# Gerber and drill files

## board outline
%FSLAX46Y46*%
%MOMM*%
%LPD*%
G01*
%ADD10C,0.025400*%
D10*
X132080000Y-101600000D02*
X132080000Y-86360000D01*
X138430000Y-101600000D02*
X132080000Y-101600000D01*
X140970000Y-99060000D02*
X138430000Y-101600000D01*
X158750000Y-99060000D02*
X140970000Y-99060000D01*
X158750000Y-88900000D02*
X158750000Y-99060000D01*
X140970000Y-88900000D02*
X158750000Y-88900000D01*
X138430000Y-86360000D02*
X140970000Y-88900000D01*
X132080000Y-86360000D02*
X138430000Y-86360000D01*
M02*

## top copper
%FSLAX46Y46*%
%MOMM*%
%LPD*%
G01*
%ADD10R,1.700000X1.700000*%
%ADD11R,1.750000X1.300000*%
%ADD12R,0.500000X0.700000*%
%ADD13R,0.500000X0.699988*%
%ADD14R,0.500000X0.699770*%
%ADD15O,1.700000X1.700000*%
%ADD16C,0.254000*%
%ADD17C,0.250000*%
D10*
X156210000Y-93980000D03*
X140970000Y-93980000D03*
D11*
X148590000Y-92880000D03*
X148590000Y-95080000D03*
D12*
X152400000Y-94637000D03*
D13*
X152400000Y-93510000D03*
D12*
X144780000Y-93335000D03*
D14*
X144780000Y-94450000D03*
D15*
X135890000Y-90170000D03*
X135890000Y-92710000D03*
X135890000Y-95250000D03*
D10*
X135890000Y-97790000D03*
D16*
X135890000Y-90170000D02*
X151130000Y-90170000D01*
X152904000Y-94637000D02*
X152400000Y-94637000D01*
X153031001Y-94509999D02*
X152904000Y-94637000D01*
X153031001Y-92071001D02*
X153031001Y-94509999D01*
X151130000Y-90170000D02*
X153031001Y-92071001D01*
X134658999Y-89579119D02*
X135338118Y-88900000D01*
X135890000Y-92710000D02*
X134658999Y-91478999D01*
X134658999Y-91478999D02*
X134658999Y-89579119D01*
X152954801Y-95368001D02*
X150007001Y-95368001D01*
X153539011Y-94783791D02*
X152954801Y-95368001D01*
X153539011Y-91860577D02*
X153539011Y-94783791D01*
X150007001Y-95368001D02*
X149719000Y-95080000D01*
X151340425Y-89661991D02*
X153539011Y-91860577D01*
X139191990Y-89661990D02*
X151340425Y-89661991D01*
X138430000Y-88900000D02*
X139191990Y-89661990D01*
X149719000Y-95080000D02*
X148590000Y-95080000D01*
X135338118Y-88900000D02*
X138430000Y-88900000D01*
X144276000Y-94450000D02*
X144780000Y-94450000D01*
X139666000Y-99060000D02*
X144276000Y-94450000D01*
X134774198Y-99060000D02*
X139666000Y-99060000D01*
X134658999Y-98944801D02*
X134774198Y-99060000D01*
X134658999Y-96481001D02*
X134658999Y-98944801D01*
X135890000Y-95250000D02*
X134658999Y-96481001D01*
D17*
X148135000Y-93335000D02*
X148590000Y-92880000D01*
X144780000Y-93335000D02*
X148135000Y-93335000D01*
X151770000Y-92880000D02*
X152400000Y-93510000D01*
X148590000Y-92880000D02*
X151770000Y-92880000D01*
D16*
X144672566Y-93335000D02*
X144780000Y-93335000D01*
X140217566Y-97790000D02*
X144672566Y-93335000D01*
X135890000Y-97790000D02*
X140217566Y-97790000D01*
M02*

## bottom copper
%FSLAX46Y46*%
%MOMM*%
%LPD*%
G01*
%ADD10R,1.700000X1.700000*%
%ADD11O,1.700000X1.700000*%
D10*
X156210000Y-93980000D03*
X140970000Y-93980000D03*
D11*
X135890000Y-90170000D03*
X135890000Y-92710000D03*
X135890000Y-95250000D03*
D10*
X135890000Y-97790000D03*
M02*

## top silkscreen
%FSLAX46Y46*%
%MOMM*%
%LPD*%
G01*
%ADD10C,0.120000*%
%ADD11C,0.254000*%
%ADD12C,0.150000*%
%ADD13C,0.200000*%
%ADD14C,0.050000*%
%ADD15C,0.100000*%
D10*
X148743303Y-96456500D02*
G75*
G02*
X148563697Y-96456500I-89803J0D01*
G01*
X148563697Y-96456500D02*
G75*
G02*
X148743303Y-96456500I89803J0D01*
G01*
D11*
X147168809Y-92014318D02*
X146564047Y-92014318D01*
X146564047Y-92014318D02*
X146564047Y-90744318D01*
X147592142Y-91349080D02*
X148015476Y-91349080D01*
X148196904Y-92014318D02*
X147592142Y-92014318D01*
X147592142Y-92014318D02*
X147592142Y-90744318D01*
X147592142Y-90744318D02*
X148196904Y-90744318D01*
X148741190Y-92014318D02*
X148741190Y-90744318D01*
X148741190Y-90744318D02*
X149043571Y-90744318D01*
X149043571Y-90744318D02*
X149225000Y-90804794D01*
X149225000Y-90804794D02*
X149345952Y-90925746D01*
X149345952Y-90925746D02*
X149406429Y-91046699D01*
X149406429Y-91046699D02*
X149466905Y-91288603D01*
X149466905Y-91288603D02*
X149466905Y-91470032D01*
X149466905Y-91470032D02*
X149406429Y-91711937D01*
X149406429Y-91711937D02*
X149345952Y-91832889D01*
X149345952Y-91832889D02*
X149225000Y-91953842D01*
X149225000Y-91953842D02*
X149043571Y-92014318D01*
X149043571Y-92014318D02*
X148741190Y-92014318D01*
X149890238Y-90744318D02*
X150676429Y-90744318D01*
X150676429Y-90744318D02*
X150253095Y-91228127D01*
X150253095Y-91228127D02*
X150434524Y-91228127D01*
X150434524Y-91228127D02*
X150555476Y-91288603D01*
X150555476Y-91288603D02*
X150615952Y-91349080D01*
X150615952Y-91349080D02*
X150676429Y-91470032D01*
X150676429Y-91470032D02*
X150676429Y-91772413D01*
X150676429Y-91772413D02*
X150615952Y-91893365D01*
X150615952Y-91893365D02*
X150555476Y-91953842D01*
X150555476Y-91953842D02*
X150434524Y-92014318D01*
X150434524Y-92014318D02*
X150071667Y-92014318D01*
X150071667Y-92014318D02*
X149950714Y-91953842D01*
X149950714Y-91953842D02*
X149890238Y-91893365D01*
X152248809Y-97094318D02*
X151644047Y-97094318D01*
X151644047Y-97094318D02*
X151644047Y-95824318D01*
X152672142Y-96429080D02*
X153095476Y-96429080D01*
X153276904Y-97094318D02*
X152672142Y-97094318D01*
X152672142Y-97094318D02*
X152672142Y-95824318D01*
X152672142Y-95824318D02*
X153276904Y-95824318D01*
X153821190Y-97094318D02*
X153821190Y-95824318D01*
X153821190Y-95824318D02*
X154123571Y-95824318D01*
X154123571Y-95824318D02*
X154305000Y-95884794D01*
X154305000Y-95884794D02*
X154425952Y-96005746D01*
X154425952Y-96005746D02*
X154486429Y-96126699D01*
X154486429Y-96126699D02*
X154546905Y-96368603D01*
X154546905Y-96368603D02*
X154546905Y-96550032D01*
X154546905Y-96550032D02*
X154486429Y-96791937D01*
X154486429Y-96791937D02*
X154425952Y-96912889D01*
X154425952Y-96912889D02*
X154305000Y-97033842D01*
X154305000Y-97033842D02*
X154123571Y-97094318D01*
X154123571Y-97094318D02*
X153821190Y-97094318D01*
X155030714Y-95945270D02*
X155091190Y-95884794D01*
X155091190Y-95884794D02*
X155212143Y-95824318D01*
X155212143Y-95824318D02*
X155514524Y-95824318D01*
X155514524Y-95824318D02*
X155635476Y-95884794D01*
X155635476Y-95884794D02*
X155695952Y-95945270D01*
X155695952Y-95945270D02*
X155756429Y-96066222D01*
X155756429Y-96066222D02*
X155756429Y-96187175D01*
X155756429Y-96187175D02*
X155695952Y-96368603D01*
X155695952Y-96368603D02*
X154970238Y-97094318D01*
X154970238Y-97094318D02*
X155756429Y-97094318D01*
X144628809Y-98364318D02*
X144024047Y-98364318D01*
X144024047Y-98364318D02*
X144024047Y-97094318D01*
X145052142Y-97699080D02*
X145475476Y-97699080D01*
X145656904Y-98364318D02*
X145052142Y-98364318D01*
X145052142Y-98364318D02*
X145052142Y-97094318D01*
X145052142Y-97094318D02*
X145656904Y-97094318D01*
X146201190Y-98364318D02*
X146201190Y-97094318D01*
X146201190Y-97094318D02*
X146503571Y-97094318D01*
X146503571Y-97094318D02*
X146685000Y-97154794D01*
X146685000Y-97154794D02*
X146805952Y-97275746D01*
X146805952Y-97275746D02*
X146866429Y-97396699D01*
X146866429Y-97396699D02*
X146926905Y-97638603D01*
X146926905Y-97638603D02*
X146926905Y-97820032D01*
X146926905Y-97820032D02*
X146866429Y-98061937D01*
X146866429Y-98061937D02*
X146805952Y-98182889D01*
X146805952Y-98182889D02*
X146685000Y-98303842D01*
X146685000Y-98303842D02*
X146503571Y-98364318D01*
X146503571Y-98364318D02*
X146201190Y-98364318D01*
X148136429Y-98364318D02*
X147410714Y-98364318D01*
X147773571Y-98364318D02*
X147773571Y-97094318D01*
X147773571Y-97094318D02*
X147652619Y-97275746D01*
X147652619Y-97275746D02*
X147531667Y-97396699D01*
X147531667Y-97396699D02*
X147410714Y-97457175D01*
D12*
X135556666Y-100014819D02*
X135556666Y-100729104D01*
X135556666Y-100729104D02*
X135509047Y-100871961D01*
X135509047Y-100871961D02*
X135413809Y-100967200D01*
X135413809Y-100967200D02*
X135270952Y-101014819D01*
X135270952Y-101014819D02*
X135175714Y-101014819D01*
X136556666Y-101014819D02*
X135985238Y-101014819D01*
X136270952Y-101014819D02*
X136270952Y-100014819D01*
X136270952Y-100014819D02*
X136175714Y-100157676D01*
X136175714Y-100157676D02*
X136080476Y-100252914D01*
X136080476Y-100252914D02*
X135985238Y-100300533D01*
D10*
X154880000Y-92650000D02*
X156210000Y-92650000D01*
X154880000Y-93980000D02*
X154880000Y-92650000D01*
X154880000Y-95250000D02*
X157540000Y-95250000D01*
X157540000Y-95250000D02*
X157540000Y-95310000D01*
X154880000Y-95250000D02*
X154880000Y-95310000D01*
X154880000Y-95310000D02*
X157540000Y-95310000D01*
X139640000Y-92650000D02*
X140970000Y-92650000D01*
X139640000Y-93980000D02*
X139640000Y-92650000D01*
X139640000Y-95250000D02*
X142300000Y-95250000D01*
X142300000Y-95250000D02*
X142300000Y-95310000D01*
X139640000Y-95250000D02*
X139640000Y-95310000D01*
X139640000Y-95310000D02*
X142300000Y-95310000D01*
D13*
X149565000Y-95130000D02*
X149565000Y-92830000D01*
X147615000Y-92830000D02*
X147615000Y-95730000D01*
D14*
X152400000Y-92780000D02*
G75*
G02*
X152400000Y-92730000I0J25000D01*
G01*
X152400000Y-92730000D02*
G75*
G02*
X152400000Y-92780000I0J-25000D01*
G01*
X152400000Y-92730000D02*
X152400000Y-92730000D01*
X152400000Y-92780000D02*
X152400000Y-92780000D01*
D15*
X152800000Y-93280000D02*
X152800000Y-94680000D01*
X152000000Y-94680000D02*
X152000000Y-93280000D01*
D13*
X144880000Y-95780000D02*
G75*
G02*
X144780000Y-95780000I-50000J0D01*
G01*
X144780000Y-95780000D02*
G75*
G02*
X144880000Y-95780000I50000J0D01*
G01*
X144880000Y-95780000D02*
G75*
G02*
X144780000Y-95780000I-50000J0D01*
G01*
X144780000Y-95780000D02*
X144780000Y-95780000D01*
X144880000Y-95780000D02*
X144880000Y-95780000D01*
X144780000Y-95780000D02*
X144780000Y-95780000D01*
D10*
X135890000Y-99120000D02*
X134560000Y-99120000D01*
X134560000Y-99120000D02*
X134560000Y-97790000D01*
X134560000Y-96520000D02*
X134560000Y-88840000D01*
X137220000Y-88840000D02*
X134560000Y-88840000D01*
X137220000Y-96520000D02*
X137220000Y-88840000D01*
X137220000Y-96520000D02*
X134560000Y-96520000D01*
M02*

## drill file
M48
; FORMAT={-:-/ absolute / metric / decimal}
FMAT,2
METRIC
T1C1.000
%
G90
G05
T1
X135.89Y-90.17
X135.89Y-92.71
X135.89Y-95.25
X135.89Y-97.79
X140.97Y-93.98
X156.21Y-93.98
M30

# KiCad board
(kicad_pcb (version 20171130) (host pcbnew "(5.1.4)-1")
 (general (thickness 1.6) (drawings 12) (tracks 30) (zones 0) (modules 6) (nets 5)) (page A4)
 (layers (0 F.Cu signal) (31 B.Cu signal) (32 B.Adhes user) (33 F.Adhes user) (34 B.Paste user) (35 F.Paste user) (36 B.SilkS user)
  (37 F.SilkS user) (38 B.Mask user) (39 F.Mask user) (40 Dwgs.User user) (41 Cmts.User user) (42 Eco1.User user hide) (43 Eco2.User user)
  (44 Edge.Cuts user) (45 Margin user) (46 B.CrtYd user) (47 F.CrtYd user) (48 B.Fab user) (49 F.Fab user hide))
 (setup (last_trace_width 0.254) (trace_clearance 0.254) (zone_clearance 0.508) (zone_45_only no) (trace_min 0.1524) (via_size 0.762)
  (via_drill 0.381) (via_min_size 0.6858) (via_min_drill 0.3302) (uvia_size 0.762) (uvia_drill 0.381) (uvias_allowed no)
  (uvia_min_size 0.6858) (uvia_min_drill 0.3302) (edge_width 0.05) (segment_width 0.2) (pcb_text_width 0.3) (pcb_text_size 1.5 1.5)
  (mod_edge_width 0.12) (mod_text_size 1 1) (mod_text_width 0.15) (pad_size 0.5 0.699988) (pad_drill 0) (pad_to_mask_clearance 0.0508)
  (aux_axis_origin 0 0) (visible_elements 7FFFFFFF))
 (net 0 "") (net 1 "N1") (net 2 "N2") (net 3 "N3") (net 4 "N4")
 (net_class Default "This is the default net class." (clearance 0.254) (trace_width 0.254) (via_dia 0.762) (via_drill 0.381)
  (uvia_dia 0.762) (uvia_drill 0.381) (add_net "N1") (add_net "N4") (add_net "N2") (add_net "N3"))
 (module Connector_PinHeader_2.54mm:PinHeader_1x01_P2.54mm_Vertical (layer F.Cu) (at 156.21 93.98)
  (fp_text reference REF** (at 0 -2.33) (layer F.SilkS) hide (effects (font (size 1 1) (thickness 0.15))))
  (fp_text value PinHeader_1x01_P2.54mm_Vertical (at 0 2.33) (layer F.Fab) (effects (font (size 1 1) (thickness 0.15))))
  (fp_line (start -1.33 -1.33) (end 0 -1.33) (layer F.SilkS) (width 0.12))
  (fp_line (start -1.33 0) (end -1.33 -1.33) (layer F.SilkS) (width 0.12))
  (fp_line (start -1.33 1.27) (end 1.33 1.27) (layer F.SilkS) (width 0.12))
  (fp_line (start 1.33 1.27) (end 1.33 1.33) (layer F.SilkS) (width 0.12))
  (fp_line (start -1.33 1.27) (end -1.33 1.33) (layer F.SilkS) (width 0.12))
  (fp_line (start -1.33 1.33) (end 1.33 1.33) (layer F.SilkS) (width 0.12))
  (pad 1 thru_hole rect (at 0 0) (size 1.7 1.7) (drill 1) (layers *.Cu *.Mask)))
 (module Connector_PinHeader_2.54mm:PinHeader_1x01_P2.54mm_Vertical (layer F.Cu) (at 140.97 93.98)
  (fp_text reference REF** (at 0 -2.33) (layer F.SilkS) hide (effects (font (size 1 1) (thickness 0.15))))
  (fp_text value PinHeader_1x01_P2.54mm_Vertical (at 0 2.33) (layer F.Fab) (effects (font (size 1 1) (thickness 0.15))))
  (fp_line (start -1.33 -1.33) (end 0 -1.33) (layer F.SilkS) (width 0.12))
  (fp_line (start -1.33 0) (end -1.33 -1.33) (layer F.SilkS) (width 0.12))
  (fp_line (start -1.33 1.27) (end 1.33 1.27) (layer F.SilkS) (width 0.12))
  (fp_line (start 1.33 1.27) (end 1.33 1.33) (layer F.SilkS) (width 0.12))
  (fp_line (start -1.33 1.27) (end -1.33 1.33) (layer F.SilkS) (width 0.12))
  (fp_line (start -1.33 1.33) (end 1.33 1.33) (layer F.SilkS) (width 0.12))
  (pad 1 thru_hole rect (at 0 0) (size 1.7 1.7) (drill 1) (layers *.Cu *.Mask)))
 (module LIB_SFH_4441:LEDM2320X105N (layer F.Cu) (at 148.59 93.98 90)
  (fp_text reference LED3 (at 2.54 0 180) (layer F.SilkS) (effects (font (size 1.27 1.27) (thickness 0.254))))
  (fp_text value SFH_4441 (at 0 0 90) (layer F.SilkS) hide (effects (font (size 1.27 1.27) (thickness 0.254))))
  (fp_line (start -1.15 0.975) (end 1.15 0.975) (layer F.SilkS) (width 0.2))
  (fp_line (start 1.15 -0.975) (end -1.75 -0.975) (layer F.SilkS) (width 0.2))
  (pad 2 smd rect (at 1.1 0 90) (size 1.3 1.75) (layers F.Cu F.Paste F.Mask) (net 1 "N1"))
  (pad 1 smd rect (at -1.1 0 90) (size 1.3 1.75) (layers F.Cu F.Paste F.Mask) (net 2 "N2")))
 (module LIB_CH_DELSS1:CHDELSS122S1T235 (layer F.Cu) (at 152.4 93.98 90)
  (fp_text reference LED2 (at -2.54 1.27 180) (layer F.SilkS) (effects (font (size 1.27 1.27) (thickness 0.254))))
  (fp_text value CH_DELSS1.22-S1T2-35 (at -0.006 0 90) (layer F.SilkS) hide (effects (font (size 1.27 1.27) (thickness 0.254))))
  (fp_arc (start 1.225 0) (end 1.25 0) (angle -180) (layer F.SilkS) (width 0.05))
  (fp_arc (start 1.225 0) (end 1.2 0) (angle -180) (layer F.SilkS) (width 0.05))
  (fp_line (start 1.25 0) (end 1.25 0) (layer F.SilkS) (width 0.05))
  (fp_line (start 1.2 0) (end 1.2 0) (layer F.SilkS) (width 0.05))
  (fp_line (start 0.7 0.4) (end -0.7 0.4) (layer F.SilkS) (width 0.1))
  (fp_line (start -0.7 -0.4) (end 0.7 -0.4) (layer F.SilkS) (width 0.1))
  (pad 2 smd rect (at -0.657 0 180) (size 0.5 0.7) (layers F.Cu F.Paste F.Mask) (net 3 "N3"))
  (pad 1 smd rect (at 0.47 0 180) (size 0.5 0.699988) (layers F.Cu F.Paste F.Mask) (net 1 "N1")))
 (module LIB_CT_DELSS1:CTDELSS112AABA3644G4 (layer F.Cu) (at 144.78 93.98)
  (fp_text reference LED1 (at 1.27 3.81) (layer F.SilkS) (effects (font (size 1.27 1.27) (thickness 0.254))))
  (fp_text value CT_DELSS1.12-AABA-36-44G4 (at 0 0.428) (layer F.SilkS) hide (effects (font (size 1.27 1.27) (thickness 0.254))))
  (fp_arc (start 0.05 1.8) (end 0 1.8) (angle -180) (layer F.SilkS) (width 0.2))
  (fp_arc (start 0.05 1.8) (end 0.1 1.8) (angle -180) (layer F.SilkS) (width 0.2))
  (fp_arc (start 0.05 1.8) (end 0 1.8) (angle -180) (layer F.SilkS) (width 0.2))
  (fp_line (start 0 1.8) (end 0 1.8) (layer F.SilkS) (width 0.2))
  (fp_line (start 0.1 1.8) (end 0.1 1.8) (layer F.SilkS) (width 0.2))
  (fp_line (start 0 1.8) (end 0 1.8) (layer F.SilkS) (width 0.2))
  (pad 2 smd rect (at 0 -0.645) (size 0.5 0.7) (layers F.Cu F.Paste F.Mask) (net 1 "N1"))
  (pad 1 smd rect (at 0 0.47) (size 0.5 0.69977) (layers F.Cu F.Paste F.Mask) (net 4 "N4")))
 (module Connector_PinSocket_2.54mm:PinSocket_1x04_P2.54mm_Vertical (layer F.Cu) (at 135.89 97.79 180)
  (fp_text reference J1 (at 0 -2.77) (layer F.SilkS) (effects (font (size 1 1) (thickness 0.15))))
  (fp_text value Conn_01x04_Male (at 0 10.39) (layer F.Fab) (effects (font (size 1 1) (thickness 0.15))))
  (fp_line (start 0 -1.33) (end 1.33 -1.33) (layer F.SilkS) (width 0.12))
  (fp_line (start 1.33 -1.33) (end 1.33 0) (layer F.SilkS) (width 0.12))
  (fp_line (start 1.33 1.27) (end 1.33 8.95) (layer F.SilkS) (width 0.12))
  (fp_line (start -1.33 8.95) (end 1.33 8.95) (layer F.SilkS) (width 0.12))
  (fp_line (start -1.33 1.27) (end -1.33 8.95) (layer F.SilkS) (width 0.12))
  (fp_line (start -1.33 1.27) (end 1.33 1.27) (layer F.SilkS) (width 0.12))
  (pad 4 thru_hole oval (at 0 7.62 180) (size 1.7 1.7) (drill 1) (layers *.Cu *.Mask) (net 3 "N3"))
  (pad 3 thru_hole oval (at 0 5.08 180) (size 1.7 1.7) (drill 1) (layers *.Cu *.Mask) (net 2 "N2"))
  (pad 2 thru_hole oval (at 0 2.54 180) (size 1.7 1.7) (drill 1) (layers *.Cu *.Mask) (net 4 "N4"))
  (pad 1 thru_hole rect (at 0 0 180) (size 1.7 1.7) (drill 1) (layers *.Cu *.Mask) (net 1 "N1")))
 (gr_circle (center 148.6535 96.4565) (end 148.717 96.52) (layer F.SilkS) (width 0.12))
 (gr_line (start 132.08 101.6) (end 132.08 86.36) (layer Edge.Cuts) (width 0.0254))
 (gr_line (start 138.43 101.6) (end 132.08 101.6) (layer Edge.Cuts) (width 0.0254))
 (gr_line (start 140.97 99.06) (end 138.43 101.6) (layer Edge.Cuts) (width 0.0254))
 (gr_line (start 158.75 99.06) (end 140.97 99.06) (layer Edge.Cuts) (width 0.0254))
 (gr_line (start 158.75 88.9) (end 158.75 99.06) (layer Edge.Cuts) (width 0.0254))
 (gr_line (start 140.97 88.9) (end 158.75 88.9) (layer Edge.Cuts) (width 0.0254))
 (gr_line (start 138.43 86.36) (end 140.97 88.9) (layer Edge.Cuts) (width 0.0254))
 (gr_line (start 132.08 86.36) (end 138.43 86.36) (layer Edge.Cuts) (width 0.0254))
 (segment (start 135.89 90.17) (end 151.13 90.17) (width 0.254) (layer F.Cu) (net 3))
 (segment (start 152.904 94.637) (end 152.4 94.637) (width 0.254) (layer F.Cu) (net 3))
 (segment (start 153.031001 94.509999) (end 152.904 94.637) (width 0.254) (layer F.Cu) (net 3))
 (segment (start 153.031001 92.071001) (end 153.031001 94.509999) (width 0.254) (layer F.Cu) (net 3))
 (segment (start 151.13 90.17) (end 153.031001 92.071001) (width 0.254) (layer F.Cu) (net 3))
 (segment (start 134.658999 89.579119) (end 135.338118 88.9) (width 0.254) (layer F.Cu) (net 2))
 (segment (start 135.89 92.71) (end 134.658999 91.478999) (width 0.254) (layer F.Cu) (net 2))
 (segment (start 134.658999 91.478999) (end 134.658999 89.579119) (width 0.254) (layer F.Cu) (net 2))
 (segment (start 152.954801 95.368001) (end 150.007001 95.368001) (width 0.254) (layer F.Cu) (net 2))
 (segment (start 153.539011 94.783791) (end 152.954801 95.368001) (width 0.254) (layer F.Cu) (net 2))
 (segment (start 153.539011 91.860577) (end 153.539011 94.783791) (width 0.254) (layer F.Cu) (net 2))
 (segment (start 150.007001 95.368001) (end 149.719 95.08) (width 0.254) (layer F.Cu) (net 2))
 (segment (start 151.340425 89.661991) (end 153.539011 91.860577) (width 0.254) (layer F.Cu) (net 2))
 (segment (start 139.19199 89.66199) (end 151.340425 89.661991) (width 0.254) (layer F.Cu) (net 2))
 (segment (start 138.43 88.9) (end 139.19199 89.66199) (width 0.254) (layer F.Cu) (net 2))
 (segment (start 149.719 95.08) (end 148.59 95.08) (width 0.254) (layer F.Cu) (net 2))
 (segment (start 135.338118 88.9) (end 138.43 88.9) (width 0.254) (layer F.Cu) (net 2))
 (segment (start 144.276 94.45) (end 144.78 94.45) (width 0.254) (layer F.Cu) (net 4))
 (segment (start 139.666 99.06) (end 144.276 94.45) (width 0.254) (layer F.Cu) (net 4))
 (segment (start 134.774198 99.06) (end 139.666 99.06) (width 0.254) (layer F.Cu) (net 4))
 (segment (start 134.658999 98.944801) (end 134.774198 99.06) (width 0.254) (layer F.Cu) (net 4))
 (segment (start 134.658999 96.481001) (end 134.658999 98.944801) (width 0.254) (layer F.Cu) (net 4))
 (segment (start 135.89 95.25) (end 134.658999 96.481001) (width 0.254) (layer F.Cu) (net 4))
 (segment (start 148.135 93.335) (end 148.59 92.88) (width 0.25) (layer F.Cu) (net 1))
 (segment (start 144.78 93.335) (end 148.135 93.335) (width 0.25) (layer F.Cu) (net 1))
 (segment (start 151.77 92.88) (end 152.4 93.51) (width 0.25) (layer F.Cu) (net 1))
 (segment (start 148.59 92.88) (end 151.77 92.88) (width 0.25) (layer F.Cu) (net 1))
 (segment (start 144.672566 93.335) (end 144.78 93.335) (width 0.254) (layer F.Cu) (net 1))
 (segment (start 140.217566 97.79) (end 144.672566 93.335) (width 0.254) (layer F.Cu) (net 1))
 (segment (start 135.89 97.79) (end 140.217566 97.79) (width 0.254) (layer F.Cu) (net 1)))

